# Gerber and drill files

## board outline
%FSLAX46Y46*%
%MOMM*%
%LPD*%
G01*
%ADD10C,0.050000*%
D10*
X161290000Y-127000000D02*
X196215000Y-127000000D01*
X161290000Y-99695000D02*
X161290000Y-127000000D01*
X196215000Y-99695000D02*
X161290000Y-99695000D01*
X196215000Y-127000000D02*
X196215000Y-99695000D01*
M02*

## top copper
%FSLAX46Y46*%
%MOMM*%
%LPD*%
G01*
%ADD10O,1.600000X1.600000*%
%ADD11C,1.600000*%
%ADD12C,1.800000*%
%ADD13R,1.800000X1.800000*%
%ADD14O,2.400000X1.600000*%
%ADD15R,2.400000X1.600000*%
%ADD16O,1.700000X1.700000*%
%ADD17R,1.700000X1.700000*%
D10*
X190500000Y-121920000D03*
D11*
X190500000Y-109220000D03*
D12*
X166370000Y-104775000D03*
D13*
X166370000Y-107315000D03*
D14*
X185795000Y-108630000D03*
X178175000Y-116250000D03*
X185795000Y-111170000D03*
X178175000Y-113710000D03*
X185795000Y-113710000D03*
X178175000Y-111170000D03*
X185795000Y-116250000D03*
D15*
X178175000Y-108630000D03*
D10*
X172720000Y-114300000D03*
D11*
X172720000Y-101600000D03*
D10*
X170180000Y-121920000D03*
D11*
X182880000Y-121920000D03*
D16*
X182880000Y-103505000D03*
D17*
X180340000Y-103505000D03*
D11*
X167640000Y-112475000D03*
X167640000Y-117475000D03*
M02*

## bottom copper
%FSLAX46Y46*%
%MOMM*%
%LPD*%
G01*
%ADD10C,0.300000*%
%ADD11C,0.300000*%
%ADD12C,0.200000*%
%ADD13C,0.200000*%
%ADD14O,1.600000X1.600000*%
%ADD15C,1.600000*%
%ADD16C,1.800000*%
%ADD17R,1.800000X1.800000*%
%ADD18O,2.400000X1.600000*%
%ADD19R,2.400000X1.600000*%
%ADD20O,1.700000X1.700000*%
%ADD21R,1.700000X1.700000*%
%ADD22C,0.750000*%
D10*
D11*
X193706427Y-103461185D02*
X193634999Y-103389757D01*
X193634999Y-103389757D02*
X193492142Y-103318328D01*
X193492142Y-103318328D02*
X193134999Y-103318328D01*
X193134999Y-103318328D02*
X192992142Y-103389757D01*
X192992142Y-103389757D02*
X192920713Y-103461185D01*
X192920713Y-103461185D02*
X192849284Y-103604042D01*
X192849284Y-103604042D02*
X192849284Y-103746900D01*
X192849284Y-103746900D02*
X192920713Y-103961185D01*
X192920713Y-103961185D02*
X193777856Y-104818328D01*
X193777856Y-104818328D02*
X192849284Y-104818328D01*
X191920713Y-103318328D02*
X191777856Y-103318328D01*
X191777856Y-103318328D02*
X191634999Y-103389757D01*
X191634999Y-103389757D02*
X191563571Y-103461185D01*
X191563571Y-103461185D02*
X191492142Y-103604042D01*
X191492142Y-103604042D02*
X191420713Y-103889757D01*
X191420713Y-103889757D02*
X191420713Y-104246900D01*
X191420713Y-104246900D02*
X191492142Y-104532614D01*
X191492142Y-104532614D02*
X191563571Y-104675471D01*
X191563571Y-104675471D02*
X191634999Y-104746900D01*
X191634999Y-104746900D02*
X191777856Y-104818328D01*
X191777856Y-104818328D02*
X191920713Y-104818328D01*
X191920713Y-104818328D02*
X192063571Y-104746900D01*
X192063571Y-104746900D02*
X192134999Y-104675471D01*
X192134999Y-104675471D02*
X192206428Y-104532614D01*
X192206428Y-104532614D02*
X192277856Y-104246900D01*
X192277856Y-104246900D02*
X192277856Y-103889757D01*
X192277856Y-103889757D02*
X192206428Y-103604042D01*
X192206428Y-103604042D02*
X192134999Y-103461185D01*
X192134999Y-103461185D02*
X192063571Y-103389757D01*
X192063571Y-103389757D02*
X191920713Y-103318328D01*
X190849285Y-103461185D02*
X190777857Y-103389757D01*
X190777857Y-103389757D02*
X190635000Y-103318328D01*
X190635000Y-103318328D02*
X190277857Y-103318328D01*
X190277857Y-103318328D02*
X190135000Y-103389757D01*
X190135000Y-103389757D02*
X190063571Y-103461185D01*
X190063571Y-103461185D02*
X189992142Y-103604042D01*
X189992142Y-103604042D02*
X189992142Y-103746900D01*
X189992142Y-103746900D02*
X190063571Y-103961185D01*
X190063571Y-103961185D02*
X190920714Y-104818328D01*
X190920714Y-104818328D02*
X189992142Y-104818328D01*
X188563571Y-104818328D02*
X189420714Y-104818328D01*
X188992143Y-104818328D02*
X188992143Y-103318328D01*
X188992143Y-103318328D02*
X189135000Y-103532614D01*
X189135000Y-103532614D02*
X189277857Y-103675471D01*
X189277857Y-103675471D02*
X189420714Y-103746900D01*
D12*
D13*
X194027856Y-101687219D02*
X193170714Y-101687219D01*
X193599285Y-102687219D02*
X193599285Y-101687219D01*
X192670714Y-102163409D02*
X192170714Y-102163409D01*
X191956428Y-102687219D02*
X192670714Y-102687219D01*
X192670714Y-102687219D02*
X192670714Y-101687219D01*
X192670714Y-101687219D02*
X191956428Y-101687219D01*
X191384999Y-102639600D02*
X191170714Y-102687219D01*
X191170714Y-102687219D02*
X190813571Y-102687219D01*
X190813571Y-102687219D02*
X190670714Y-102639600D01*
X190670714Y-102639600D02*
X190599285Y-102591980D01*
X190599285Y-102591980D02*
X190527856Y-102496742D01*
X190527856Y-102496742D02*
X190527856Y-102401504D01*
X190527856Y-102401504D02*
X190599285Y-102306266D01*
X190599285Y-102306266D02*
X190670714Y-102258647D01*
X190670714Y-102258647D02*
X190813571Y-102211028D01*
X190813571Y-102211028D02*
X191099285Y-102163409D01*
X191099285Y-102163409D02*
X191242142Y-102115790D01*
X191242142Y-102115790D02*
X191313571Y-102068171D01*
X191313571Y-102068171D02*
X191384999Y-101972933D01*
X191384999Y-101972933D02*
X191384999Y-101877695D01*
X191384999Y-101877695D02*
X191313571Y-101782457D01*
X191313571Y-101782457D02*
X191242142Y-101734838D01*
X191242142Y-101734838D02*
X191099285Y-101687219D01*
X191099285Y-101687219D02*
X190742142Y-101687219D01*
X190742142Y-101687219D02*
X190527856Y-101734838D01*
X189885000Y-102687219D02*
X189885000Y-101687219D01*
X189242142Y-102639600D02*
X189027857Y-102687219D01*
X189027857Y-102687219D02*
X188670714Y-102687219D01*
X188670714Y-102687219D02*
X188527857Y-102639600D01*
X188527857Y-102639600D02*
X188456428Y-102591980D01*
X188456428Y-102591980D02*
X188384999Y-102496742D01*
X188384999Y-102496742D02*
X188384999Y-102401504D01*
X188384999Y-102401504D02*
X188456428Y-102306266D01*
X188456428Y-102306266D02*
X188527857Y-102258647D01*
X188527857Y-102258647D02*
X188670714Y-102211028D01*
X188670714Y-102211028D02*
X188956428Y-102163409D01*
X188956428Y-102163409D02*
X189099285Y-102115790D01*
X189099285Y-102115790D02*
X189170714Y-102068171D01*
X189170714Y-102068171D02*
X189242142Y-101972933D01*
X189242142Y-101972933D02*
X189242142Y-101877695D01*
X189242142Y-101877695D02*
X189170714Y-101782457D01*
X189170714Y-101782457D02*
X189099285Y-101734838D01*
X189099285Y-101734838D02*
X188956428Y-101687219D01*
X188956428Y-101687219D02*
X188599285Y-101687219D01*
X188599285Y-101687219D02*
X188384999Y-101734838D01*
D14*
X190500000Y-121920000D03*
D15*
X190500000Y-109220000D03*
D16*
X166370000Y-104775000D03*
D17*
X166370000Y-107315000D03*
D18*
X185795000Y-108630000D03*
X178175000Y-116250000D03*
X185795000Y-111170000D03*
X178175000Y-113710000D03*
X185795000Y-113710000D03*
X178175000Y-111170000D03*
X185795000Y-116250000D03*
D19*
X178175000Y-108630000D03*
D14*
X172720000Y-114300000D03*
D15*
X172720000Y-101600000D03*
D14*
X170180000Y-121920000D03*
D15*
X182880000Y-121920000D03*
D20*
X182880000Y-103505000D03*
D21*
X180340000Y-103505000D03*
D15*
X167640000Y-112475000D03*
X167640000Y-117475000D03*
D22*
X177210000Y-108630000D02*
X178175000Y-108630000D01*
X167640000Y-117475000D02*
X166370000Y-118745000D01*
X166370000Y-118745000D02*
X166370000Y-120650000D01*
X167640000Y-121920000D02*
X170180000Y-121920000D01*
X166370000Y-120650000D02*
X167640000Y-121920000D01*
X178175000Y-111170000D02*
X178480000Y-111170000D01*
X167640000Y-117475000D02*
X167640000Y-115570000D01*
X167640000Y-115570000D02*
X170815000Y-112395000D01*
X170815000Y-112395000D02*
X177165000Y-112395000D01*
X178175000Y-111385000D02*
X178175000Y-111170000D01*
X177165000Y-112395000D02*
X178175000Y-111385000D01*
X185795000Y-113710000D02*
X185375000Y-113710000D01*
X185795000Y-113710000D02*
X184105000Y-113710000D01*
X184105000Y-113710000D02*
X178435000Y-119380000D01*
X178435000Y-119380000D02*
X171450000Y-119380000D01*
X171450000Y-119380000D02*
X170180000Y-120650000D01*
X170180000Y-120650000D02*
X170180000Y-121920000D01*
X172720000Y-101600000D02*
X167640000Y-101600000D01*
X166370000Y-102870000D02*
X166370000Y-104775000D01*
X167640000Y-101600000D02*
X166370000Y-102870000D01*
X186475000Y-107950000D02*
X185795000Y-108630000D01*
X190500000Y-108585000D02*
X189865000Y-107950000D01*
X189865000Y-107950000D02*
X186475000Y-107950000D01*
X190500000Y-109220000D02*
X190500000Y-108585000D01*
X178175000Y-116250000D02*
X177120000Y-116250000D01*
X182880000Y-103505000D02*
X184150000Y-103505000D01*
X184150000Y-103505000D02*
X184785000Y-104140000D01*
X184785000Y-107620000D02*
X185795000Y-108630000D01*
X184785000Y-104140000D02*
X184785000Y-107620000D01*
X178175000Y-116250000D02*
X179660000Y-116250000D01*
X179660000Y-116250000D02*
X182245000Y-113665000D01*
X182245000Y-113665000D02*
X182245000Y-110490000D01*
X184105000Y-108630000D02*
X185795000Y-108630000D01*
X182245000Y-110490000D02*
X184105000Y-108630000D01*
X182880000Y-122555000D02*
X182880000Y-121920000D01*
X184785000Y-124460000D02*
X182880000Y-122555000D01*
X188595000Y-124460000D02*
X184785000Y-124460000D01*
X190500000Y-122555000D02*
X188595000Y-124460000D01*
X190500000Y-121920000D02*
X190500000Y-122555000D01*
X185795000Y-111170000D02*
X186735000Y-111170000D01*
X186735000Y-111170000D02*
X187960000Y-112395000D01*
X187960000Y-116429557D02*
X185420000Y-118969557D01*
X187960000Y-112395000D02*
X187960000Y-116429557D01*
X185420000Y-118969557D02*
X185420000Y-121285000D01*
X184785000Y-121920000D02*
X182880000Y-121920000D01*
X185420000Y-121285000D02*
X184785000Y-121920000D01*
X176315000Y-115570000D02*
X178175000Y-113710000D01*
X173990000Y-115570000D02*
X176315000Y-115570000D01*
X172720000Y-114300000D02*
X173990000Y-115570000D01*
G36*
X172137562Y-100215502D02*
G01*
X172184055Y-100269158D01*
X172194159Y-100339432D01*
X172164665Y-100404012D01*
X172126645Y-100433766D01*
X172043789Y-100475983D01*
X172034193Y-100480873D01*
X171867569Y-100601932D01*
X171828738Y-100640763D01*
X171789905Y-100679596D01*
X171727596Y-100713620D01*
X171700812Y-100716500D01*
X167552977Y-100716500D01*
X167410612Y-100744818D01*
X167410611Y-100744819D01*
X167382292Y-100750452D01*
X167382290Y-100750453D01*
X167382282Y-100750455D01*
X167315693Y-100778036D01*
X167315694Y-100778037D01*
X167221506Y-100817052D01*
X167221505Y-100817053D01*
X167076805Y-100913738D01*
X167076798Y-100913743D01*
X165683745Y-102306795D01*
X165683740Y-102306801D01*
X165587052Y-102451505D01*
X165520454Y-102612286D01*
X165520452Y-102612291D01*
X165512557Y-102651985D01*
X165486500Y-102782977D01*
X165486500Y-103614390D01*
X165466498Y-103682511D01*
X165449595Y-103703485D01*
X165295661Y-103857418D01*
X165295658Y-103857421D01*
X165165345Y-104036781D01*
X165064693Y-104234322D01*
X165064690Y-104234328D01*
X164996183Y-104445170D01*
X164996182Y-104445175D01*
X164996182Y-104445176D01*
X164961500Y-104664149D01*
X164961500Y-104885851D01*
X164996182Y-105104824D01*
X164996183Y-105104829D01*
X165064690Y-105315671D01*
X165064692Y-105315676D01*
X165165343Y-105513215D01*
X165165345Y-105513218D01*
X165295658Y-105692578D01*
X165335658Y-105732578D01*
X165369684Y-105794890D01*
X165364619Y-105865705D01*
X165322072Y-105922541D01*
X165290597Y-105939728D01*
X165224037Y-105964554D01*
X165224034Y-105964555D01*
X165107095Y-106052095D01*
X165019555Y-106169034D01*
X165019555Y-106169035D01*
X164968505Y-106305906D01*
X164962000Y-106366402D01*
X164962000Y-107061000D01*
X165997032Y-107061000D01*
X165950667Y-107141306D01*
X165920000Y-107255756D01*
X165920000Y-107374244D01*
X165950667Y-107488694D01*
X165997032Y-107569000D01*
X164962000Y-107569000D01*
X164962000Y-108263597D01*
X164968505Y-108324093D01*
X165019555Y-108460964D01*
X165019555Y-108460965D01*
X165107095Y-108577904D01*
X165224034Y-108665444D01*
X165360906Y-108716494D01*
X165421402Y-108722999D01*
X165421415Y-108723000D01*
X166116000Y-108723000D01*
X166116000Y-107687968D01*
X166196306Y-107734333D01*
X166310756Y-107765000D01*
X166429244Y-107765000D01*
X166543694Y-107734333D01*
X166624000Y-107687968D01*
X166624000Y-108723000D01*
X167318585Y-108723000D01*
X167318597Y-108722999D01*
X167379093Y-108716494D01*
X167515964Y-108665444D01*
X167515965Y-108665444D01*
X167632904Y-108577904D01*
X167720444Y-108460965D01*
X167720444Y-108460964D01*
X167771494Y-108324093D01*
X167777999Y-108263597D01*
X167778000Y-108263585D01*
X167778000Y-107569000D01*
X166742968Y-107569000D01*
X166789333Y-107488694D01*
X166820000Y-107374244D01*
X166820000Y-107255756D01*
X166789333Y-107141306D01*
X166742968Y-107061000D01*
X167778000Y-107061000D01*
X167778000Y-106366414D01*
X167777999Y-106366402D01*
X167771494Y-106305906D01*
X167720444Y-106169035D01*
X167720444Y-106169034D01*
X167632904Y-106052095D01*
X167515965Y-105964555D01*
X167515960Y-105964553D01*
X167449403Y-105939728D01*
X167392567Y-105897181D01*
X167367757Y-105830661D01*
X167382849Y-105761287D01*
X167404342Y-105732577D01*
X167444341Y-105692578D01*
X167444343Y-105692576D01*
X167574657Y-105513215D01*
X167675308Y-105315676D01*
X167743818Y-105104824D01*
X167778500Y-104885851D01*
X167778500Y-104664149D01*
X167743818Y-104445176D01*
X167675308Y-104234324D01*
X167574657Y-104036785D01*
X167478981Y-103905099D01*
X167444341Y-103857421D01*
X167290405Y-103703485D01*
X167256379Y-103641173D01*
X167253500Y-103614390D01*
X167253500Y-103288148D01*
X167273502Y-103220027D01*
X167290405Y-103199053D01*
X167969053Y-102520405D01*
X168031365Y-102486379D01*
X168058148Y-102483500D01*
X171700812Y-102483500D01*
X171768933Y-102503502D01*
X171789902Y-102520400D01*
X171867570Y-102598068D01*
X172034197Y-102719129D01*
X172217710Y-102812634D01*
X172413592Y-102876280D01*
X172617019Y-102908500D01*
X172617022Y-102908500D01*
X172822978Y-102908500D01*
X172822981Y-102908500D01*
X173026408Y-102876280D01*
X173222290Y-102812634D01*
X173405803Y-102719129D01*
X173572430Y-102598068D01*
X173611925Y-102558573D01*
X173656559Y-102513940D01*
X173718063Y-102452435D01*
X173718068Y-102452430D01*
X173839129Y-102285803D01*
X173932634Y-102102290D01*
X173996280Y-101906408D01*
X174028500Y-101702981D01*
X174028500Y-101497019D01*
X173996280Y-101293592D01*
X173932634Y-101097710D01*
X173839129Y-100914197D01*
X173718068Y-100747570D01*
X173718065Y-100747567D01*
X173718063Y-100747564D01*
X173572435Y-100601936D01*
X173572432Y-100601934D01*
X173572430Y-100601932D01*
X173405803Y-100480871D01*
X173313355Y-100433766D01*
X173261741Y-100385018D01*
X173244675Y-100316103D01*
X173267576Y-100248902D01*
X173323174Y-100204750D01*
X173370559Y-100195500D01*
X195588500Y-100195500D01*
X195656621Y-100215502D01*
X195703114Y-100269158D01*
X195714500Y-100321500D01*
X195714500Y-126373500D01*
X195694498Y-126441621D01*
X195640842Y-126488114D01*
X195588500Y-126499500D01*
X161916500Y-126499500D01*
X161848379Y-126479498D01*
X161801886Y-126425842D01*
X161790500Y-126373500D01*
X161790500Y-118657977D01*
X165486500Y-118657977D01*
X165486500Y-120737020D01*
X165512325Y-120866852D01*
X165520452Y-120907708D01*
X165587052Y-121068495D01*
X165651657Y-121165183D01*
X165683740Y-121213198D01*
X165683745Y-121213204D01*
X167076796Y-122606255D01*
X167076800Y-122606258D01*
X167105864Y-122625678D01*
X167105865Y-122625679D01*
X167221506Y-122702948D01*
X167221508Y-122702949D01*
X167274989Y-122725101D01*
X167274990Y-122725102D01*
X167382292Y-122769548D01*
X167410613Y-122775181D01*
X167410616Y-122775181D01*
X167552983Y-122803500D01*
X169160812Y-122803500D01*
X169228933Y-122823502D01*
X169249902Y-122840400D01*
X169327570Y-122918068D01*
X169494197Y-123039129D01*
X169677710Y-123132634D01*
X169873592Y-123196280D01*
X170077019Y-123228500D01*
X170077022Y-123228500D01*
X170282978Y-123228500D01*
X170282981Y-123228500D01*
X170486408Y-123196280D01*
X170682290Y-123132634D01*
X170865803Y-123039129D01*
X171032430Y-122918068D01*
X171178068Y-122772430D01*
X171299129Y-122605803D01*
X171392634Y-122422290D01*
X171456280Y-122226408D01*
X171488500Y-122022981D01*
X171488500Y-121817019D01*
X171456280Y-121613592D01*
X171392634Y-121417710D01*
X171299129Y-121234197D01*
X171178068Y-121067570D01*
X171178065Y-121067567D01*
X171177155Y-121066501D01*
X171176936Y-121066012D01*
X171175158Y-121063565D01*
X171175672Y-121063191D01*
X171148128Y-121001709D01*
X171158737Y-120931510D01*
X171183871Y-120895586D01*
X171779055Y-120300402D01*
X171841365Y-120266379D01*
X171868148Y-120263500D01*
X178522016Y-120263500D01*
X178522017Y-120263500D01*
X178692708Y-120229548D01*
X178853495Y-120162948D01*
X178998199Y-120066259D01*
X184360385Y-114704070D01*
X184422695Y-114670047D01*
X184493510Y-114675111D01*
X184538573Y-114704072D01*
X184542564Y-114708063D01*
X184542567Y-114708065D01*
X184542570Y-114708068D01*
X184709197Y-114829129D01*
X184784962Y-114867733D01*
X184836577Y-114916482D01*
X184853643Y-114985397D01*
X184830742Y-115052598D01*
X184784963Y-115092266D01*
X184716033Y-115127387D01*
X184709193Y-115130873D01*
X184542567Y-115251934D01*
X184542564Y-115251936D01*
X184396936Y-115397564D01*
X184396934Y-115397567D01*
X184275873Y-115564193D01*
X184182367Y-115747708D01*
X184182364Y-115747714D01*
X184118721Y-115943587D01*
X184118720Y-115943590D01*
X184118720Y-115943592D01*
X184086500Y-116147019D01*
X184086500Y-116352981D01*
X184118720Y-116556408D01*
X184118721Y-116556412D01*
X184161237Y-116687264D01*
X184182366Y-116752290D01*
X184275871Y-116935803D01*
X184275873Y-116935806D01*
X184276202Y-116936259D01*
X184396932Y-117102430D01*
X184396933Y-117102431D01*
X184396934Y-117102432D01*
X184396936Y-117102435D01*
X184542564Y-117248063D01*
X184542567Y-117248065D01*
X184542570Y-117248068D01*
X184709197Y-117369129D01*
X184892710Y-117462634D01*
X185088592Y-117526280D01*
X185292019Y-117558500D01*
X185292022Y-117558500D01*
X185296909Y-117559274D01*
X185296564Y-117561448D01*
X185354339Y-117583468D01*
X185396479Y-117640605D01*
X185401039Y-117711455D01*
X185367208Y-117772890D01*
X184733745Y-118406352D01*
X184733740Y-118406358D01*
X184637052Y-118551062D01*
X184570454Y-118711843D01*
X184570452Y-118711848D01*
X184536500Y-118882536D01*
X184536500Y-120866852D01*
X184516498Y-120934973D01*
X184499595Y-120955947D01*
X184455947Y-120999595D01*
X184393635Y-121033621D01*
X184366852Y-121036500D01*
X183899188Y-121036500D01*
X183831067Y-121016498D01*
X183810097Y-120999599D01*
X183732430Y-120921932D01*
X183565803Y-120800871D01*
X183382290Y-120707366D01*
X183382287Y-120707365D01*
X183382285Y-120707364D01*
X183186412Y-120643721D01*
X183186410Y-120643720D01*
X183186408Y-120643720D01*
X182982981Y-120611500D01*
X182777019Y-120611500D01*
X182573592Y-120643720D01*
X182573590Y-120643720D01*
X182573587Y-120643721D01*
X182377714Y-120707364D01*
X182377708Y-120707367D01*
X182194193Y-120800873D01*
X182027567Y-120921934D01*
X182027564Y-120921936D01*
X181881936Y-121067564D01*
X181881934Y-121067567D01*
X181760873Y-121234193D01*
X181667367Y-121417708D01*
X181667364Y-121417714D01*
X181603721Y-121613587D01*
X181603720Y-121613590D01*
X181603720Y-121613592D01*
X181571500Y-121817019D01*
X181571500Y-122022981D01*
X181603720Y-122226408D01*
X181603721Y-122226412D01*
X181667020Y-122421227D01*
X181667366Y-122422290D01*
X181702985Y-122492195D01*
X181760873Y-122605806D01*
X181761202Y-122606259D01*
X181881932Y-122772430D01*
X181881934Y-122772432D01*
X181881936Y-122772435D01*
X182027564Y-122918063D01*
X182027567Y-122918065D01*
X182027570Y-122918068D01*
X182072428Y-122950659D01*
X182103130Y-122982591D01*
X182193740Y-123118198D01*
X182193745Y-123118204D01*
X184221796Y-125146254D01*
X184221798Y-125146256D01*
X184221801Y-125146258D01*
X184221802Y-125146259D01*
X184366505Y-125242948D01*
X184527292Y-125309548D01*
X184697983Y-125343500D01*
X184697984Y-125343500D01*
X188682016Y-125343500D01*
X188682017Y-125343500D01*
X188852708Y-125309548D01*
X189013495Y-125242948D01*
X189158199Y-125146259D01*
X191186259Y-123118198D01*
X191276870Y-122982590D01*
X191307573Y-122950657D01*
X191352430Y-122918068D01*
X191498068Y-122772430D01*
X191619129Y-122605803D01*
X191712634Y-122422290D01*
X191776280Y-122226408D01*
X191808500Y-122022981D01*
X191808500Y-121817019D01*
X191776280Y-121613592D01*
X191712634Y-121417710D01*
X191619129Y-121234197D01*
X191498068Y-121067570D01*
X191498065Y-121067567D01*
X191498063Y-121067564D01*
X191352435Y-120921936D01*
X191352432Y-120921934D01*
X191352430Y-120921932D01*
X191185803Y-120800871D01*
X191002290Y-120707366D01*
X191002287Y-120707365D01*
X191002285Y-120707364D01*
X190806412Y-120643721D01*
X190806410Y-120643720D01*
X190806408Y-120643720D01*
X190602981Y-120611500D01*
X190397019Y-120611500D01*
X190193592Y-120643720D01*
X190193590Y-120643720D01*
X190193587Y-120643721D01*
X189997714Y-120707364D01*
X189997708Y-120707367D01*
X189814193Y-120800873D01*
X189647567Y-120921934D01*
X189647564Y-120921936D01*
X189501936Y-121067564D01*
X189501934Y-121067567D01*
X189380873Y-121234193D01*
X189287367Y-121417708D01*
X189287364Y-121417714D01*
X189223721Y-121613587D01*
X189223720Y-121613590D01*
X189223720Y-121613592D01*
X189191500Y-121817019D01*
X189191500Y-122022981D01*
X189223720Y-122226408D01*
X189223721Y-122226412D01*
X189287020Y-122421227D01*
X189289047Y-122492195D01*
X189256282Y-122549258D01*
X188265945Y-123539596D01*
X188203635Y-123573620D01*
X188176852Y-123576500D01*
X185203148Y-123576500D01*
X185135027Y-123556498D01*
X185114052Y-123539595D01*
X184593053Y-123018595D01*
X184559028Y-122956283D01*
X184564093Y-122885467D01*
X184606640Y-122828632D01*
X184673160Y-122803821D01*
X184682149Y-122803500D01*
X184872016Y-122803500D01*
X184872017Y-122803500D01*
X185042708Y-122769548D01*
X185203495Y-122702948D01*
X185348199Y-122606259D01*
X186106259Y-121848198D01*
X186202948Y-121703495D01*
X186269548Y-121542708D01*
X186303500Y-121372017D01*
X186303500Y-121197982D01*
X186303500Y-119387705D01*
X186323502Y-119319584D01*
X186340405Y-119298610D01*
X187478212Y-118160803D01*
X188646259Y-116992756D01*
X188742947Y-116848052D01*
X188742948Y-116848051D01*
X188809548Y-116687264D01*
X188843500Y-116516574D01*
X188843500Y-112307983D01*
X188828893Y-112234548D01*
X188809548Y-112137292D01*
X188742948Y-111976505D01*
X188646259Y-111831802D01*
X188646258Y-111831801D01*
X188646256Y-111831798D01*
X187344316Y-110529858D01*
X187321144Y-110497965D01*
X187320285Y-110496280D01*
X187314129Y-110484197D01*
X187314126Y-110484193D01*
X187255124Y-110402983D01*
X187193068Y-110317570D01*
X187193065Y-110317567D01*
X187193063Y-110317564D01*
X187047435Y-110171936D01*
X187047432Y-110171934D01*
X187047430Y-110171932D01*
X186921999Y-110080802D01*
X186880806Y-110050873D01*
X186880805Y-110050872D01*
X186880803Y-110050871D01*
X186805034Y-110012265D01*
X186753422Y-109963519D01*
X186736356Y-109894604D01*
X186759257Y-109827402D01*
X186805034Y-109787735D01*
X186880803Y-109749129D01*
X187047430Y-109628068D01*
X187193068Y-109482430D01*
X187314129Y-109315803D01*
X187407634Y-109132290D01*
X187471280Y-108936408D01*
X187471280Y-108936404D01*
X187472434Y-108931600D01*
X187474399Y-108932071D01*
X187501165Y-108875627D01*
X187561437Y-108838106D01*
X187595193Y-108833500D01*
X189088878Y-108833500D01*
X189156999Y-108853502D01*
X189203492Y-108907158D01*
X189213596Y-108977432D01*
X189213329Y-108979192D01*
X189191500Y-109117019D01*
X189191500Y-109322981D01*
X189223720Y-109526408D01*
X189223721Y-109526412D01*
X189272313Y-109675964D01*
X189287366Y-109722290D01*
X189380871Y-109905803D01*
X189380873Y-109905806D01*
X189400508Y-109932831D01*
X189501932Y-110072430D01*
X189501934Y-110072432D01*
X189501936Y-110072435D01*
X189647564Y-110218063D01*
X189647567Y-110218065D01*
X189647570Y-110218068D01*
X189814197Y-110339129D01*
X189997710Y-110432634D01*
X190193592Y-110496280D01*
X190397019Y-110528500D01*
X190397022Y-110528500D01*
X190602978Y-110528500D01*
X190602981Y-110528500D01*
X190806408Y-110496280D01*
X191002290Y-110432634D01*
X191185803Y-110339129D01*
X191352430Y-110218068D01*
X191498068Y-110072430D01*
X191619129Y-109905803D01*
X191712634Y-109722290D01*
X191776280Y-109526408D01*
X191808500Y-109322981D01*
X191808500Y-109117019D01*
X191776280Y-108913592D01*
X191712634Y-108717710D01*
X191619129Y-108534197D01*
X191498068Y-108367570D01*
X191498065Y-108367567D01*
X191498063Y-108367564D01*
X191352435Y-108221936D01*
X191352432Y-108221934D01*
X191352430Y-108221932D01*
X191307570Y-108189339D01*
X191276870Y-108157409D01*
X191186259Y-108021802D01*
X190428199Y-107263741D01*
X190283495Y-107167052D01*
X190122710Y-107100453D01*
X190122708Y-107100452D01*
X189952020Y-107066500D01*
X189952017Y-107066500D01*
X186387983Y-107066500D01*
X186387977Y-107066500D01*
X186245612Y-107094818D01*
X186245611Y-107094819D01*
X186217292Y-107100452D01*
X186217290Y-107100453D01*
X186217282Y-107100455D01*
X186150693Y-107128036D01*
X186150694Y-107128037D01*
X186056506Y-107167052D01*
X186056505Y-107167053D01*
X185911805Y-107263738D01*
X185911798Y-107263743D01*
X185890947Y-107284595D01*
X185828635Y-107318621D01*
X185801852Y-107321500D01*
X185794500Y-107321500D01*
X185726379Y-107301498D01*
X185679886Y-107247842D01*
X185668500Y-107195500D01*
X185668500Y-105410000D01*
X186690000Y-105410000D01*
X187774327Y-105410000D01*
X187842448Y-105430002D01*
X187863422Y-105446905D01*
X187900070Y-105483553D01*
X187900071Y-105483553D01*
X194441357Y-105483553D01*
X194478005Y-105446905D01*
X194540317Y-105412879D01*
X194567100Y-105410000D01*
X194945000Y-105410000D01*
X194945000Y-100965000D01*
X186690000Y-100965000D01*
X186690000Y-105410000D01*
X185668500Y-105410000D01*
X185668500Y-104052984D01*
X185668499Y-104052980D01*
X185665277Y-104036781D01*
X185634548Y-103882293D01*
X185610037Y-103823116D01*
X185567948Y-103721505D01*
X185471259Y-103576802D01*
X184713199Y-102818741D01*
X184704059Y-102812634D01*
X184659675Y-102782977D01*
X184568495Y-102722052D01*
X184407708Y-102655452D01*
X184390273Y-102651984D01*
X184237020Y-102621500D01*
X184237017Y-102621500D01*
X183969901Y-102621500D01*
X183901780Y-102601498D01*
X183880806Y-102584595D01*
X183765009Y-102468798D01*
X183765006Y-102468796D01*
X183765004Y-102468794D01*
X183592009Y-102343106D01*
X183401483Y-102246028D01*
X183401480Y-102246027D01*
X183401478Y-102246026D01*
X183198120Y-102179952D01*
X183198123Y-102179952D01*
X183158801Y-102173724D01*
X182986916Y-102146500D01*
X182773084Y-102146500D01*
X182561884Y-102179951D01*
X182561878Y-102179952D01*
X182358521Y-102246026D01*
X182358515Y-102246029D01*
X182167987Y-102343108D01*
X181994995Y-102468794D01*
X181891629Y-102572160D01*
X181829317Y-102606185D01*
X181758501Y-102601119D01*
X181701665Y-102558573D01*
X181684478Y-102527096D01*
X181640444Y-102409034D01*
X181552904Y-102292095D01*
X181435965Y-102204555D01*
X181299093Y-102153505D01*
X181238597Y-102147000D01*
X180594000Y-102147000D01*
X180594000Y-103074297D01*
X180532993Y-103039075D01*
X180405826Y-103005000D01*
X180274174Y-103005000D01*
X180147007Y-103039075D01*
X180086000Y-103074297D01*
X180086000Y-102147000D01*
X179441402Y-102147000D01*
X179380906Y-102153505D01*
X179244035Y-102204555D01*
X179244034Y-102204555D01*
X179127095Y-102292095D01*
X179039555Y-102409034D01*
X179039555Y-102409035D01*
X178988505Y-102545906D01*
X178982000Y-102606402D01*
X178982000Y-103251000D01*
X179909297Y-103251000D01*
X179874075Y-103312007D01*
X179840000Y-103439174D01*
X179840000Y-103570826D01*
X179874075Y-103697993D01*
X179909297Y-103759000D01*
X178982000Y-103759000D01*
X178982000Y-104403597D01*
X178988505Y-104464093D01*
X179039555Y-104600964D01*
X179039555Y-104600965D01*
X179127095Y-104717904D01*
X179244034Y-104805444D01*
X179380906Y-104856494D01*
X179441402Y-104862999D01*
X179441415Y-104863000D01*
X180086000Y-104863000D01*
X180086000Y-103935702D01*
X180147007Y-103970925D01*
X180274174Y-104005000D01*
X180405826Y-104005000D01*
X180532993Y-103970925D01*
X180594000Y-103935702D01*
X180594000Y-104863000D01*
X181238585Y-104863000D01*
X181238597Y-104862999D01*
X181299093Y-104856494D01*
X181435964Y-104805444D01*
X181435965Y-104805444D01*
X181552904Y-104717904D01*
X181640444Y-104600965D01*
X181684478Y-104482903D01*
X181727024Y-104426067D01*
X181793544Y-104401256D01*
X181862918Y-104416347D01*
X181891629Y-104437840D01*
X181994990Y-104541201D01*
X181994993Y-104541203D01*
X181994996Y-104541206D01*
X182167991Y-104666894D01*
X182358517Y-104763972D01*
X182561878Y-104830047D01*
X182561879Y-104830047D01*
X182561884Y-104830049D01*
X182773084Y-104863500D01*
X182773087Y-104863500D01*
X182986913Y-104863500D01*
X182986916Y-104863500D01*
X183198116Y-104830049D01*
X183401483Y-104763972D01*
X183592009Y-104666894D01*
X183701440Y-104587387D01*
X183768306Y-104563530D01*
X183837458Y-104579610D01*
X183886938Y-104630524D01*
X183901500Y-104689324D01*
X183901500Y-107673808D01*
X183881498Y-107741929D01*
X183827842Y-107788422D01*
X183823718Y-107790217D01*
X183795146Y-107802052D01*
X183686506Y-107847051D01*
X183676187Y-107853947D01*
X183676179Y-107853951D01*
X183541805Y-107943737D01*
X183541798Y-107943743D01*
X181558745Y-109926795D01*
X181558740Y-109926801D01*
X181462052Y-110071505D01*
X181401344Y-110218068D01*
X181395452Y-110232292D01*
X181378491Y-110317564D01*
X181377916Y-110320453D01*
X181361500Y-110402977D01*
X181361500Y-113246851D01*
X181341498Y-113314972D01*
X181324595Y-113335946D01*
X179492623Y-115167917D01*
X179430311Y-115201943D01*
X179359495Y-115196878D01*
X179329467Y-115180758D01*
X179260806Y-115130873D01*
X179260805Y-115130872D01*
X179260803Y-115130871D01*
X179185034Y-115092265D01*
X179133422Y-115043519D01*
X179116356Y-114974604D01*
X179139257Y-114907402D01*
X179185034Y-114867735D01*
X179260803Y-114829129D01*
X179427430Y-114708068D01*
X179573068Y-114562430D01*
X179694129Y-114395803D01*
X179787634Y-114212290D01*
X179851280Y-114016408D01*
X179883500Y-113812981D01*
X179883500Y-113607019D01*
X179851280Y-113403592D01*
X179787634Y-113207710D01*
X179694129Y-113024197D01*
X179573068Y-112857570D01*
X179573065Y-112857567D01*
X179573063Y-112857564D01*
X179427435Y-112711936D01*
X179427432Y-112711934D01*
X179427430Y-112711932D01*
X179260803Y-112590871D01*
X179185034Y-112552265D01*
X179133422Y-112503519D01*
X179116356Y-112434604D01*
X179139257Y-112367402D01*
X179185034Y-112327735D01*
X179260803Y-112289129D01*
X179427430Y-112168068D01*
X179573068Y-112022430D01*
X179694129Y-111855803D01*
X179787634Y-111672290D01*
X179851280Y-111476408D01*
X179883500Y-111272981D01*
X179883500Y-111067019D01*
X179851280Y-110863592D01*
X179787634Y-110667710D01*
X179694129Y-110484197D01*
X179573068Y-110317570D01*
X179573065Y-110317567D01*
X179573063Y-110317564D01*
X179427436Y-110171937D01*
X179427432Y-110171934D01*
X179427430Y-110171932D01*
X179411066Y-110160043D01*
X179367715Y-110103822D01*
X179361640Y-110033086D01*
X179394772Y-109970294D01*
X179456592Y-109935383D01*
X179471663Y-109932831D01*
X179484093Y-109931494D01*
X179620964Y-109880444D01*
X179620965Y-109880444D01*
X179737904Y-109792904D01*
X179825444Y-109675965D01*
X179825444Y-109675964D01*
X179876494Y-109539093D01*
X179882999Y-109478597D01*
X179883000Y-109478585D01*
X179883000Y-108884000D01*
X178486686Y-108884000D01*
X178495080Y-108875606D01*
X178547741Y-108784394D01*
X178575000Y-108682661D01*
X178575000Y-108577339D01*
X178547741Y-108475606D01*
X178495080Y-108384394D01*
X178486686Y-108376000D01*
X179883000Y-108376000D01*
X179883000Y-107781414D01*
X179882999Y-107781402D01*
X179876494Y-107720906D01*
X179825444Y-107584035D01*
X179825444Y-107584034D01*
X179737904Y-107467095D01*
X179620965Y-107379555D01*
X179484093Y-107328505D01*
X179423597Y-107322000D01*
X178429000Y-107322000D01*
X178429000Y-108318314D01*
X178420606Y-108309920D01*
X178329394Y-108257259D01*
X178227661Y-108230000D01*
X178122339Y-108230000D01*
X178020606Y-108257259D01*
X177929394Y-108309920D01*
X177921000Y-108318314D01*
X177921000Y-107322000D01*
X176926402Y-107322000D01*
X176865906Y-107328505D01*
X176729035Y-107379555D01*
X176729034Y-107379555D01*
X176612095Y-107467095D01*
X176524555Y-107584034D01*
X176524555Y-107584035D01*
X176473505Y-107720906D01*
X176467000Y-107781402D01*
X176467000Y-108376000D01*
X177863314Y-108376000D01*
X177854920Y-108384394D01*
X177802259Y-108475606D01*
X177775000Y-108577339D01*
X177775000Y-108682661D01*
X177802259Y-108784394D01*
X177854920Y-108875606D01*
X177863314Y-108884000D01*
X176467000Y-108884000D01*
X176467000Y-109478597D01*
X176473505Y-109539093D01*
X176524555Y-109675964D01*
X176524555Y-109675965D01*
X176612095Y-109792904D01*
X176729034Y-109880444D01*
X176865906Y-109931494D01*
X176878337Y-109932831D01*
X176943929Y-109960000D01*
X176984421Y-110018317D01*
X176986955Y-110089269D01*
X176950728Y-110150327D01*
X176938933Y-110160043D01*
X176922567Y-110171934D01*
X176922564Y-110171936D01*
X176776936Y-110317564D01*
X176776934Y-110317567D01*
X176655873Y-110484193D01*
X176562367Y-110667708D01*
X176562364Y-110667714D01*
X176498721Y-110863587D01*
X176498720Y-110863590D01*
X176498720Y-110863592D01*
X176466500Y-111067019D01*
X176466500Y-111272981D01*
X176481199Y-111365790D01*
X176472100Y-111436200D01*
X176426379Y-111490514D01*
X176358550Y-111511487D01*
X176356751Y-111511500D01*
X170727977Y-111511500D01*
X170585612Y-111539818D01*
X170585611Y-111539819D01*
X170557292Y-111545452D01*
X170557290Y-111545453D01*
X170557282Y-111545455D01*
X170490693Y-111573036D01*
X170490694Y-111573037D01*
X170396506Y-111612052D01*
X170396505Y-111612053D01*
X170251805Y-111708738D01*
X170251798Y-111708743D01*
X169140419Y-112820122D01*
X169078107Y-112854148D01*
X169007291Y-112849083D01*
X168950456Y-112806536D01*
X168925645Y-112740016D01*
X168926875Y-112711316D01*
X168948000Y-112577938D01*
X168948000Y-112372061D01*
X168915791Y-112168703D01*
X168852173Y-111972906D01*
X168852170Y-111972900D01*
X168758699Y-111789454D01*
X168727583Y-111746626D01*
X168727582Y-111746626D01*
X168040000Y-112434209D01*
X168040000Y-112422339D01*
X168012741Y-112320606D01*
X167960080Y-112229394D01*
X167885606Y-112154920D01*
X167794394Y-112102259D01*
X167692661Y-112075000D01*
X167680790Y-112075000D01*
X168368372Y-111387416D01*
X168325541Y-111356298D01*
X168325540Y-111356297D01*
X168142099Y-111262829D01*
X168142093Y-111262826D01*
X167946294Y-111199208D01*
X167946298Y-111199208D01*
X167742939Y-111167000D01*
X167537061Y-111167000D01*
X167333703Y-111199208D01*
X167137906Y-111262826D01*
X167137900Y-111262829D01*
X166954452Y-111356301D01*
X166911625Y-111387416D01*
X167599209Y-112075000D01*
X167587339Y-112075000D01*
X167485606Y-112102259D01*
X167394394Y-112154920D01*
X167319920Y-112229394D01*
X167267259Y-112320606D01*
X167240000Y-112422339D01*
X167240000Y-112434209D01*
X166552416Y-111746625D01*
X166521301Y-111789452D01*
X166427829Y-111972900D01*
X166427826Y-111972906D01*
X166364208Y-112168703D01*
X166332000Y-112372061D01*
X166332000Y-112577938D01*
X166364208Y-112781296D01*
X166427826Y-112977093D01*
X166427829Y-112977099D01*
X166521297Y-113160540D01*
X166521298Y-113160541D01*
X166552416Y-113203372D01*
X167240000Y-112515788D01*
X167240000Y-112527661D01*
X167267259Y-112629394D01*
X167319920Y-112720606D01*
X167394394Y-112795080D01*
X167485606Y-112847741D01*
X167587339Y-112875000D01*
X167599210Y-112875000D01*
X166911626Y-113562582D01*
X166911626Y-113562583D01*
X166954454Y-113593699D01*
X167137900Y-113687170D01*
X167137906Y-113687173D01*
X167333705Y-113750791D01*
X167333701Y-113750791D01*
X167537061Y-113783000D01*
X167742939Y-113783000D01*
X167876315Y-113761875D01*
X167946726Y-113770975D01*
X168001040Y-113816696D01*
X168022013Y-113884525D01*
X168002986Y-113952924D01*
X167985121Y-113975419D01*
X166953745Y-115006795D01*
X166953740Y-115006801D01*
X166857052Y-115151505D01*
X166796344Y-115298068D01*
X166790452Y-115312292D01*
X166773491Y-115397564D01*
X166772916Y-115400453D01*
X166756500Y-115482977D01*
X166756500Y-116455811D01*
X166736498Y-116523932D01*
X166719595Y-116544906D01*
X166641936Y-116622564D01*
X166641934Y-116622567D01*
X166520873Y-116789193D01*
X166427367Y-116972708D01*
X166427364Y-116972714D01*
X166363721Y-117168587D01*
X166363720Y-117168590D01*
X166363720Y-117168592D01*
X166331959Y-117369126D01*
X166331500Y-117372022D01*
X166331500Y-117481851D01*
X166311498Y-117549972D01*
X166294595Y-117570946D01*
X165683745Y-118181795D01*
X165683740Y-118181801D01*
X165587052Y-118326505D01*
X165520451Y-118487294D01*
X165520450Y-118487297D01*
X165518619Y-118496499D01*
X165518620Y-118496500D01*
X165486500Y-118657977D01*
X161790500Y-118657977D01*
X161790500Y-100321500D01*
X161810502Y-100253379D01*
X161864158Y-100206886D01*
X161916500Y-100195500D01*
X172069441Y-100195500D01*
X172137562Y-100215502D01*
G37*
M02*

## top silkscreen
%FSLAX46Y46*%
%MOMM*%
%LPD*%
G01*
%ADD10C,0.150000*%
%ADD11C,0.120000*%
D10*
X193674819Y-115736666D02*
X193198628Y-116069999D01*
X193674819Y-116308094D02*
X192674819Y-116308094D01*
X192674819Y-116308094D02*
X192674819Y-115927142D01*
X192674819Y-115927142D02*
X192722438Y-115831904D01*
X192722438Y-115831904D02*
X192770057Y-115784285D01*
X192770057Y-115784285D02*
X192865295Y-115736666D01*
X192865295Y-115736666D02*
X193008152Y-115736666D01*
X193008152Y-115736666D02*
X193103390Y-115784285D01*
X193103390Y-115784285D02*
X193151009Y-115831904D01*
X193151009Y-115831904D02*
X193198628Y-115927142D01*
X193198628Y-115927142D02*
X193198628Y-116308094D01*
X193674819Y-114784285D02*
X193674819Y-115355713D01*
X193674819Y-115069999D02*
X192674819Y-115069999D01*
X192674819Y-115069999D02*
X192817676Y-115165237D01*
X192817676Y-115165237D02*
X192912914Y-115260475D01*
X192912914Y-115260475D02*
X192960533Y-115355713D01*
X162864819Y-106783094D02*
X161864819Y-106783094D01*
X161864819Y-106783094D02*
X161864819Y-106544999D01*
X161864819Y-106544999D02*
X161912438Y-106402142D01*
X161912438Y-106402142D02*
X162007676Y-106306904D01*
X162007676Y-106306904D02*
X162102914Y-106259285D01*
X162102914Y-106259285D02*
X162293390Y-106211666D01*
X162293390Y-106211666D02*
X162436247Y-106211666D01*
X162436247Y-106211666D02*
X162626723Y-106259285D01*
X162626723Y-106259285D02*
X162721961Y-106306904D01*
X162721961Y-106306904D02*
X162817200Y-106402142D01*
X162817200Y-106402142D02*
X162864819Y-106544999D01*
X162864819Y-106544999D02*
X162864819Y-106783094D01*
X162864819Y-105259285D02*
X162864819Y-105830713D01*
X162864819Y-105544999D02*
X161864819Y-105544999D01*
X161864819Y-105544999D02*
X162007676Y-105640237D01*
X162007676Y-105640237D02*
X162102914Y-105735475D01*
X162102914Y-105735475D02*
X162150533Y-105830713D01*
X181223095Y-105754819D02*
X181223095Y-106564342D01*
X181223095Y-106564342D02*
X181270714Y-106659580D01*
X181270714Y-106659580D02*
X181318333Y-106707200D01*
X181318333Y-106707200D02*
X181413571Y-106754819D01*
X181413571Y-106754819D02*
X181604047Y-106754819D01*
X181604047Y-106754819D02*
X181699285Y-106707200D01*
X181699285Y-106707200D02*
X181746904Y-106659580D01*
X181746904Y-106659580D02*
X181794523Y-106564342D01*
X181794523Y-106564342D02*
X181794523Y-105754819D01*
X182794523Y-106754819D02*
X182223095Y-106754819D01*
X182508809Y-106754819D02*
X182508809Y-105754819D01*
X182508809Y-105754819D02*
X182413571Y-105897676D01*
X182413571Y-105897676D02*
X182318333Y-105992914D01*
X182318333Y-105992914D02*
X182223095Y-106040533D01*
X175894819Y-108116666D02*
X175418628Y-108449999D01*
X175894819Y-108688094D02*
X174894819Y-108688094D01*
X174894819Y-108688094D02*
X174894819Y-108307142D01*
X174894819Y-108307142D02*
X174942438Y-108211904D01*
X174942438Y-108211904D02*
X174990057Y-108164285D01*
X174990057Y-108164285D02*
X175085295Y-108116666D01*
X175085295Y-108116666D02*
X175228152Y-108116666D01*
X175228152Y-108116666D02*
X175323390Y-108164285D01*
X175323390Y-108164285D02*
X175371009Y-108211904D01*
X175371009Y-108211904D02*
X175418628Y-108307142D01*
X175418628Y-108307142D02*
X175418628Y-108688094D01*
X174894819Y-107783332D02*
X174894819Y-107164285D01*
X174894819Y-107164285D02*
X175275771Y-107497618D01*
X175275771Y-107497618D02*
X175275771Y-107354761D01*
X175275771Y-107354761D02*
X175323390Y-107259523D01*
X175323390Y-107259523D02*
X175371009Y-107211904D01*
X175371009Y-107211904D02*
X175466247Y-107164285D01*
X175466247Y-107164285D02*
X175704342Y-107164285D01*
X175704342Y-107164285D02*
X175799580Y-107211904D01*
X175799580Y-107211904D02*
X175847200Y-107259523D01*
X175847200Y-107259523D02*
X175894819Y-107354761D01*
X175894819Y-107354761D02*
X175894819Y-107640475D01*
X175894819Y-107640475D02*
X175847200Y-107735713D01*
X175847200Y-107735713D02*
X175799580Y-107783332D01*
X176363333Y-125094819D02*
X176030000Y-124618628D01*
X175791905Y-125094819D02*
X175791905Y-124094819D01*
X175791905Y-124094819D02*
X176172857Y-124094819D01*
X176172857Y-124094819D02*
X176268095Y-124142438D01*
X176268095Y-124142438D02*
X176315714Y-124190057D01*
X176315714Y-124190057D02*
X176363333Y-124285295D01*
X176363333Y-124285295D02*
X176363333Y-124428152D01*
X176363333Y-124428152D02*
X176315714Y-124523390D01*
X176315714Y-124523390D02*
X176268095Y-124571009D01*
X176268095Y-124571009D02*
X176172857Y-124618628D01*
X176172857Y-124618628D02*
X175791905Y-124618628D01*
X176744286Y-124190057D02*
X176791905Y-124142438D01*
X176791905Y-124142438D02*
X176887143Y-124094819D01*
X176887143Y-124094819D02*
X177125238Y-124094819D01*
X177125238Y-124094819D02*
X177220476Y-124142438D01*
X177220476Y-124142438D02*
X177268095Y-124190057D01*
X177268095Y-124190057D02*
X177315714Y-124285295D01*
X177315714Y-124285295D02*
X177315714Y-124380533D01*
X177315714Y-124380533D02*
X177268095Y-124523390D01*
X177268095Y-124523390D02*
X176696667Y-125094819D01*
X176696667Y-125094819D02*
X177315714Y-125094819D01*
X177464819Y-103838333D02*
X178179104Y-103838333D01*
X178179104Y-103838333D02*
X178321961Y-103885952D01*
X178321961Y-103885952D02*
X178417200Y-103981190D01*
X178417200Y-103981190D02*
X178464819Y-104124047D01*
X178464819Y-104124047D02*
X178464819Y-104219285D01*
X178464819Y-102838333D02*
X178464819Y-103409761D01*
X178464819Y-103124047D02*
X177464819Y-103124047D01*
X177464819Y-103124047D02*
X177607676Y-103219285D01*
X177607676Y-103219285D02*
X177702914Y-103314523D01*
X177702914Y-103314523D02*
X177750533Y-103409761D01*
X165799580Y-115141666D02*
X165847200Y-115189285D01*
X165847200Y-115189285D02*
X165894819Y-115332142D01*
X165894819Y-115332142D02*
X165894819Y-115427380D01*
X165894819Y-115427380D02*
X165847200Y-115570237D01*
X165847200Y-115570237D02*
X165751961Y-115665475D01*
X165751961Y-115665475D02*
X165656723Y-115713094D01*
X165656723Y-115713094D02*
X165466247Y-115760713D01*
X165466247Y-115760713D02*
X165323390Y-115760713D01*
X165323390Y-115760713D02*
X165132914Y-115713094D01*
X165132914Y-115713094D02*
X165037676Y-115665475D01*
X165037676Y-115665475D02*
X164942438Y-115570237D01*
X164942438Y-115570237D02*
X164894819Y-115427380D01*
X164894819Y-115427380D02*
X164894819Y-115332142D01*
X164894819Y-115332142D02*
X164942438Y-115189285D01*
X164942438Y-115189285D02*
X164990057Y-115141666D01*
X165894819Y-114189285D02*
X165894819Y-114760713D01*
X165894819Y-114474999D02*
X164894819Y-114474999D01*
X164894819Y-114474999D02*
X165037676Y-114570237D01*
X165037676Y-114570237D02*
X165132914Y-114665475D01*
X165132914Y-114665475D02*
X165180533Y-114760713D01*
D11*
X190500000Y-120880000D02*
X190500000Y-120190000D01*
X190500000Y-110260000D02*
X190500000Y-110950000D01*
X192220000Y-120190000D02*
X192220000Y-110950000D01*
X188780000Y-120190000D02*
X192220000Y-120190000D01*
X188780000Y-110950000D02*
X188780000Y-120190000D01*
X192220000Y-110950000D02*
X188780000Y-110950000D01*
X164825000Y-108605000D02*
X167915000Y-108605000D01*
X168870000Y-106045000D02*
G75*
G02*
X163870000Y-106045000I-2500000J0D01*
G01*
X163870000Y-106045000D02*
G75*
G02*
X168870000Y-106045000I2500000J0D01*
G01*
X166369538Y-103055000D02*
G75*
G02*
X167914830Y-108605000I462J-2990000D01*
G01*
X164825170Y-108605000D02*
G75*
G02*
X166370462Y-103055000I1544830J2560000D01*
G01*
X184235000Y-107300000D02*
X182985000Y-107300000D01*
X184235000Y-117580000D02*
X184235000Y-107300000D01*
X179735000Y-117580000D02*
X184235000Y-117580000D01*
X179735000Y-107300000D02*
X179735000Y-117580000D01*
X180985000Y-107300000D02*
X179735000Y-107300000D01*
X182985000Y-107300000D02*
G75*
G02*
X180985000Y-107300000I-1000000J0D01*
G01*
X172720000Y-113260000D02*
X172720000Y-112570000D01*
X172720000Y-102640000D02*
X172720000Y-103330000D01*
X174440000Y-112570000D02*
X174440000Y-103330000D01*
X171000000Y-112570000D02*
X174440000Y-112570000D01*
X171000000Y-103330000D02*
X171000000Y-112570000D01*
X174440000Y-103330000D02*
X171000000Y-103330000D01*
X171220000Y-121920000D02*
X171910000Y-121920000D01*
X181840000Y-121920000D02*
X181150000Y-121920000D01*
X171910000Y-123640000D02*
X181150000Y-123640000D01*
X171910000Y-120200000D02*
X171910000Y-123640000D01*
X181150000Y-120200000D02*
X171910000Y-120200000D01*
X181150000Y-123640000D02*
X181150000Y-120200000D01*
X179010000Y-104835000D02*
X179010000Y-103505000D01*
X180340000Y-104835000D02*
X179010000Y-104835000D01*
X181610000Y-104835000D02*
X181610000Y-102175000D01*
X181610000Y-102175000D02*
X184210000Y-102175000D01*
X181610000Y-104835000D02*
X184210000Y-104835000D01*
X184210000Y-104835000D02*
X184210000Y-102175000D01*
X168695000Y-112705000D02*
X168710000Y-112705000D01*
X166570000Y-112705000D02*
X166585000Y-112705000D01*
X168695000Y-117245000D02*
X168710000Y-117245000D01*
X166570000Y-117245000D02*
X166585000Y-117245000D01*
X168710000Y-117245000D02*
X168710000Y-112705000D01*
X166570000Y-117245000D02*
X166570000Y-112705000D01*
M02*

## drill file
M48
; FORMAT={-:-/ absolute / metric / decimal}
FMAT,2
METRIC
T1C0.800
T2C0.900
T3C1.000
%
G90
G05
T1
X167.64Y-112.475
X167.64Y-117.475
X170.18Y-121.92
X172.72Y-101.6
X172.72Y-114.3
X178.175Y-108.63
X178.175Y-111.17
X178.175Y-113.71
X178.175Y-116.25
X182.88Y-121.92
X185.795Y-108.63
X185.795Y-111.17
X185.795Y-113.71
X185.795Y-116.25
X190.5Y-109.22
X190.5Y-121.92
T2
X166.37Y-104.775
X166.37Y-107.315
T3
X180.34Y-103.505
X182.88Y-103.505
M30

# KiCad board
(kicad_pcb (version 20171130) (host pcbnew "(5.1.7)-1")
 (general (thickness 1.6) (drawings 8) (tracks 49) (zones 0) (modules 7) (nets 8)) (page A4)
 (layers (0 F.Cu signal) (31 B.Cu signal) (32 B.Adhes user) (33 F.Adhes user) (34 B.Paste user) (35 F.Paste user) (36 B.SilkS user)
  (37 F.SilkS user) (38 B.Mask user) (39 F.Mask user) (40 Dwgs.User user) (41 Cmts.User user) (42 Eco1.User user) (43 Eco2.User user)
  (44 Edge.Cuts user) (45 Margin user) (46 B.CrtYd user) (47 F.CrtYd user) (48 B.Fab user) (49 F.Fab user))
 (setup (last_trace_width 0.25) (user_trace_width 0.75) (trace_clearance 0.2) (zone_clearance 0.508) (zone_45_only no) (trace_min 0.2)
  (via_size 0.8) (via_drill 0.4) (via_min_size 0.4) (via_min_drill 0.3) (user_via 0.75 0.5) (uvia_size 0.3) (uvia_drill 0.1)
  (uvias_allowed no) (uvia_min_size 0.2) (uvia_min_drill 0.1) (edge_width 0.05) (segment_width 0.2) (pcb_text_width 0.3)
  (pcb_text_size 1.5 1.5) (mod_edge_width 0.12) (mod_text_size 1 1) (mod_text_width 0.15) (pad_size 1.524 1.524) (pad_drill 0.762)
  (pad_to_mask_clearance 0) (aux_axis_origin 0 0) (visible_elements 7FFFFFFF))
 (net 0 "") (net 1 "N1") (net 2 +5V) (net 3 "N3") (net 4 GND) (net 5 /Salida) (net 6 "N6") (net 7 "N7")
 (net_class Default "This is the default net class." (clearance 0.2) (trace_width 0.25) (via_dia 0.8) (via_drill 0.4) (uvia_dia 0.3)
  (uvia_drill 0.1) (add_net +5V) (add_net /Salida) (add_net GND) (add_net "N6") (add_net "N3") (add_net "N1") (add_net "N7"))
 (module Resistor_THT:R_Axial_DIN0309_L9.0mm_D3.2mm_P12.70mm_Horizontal (layer F.Cu) (at 190.5 109.22 270)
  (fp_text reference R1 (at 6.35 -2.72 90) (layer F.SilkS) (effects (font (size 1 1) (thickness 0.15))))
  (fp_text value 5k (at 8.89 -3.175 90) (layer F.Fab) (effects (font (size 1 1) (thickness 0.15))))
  (fp_line (start 11.66 0) (end 10.97 0) (layer F.SilkS) (width 0.12))
  (fp_line (start 1.04 0) (end 1.73 0) (layer F.SilkS) (width 0.12))
  (fp_line (start 10.97 -1.72) (end 1.73 -1.72) (layer F.SilkS) (width 0.12))
  (fp_line (start 10.97 1.72) (end 10.97 -1.72) (layer F.SilkS) (width 0.12))
  (fp_line (start 1.73 1.72) (end 10.97 1.72) (layer F.SilkS) (width 0.12))
  (fp_line (start 1.73 -1.72) (end 1.73 1.72) (layer F.SilkS) (width 0.12))
  (pad 2 thru_hole oval (at 12.7 0 270) (size 1.6 1.6) (drill 0.8) (layers *.Cu *.Mask) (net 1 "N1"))
  (pad 1 thru_hole circle (at 0 0 270) (size 1.6 1.6) (drill 0.8) (layers *.Cu *.Mask) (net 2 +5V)))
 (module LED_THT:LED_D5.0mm (layer F.Cu) (at 166.37 107.315 90)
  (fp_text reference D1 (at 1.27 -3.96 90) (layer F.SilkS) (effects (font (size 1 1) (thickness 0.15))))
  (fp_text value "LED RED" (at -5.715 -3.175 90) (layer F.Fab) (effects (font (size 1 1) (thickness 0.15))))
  (fp_line (start -1.29 -1.545) (end -1.29 1.545) (layer F.SilkS) (width 0.12))
  (fp_circle (center 1.27 0) (end 3.77 0) (layer F.SilkS) (width 0.12))
  (fp_arc (start 1.27 0) (end -1.29 1.54483) (angle -148.9) (layer F.SilkS) (width 0.12))
  (fp_arc (start 1.27 0) (end -1.29 -1.54483) (angle 148.9) (layer F.SilkS) (width 0.12))
  (pad 2 thru_hole circle (at 2.54 0 90) (size 1.8 1.8) (drill 0.9) (layers *.Cu *.Mask) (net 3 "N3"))
  (pad 1 thru_hole rect (at 0 0 90) (size 1.8 1.8) (drill 0.9) (layers *.Cu *.Mask) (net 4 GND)))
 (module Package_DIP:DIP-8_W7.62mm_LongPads (layer F.Cu) (at 178.175 108.63)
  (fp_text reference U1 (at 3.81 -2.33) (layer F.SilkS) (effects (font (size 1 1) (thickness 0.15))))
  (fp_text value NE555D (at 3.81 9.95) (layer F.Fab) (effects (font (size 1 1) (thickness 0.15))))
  (fp_line (start 6.06 -1.33) (end 4.81 -1.33) (layer F.SilkS) (width 0.12))
  (fp_line (start 6.06 8.95) (end 6.06 -1.33) (layer F.SilkS) (width 0.12))
  (fp_line (start 1.56 8.95) (end 6.06 8.95) (layer F.SilkS) (width 0.12))
  (fp_line (start 1.56 -1.33) (end 1.56 8.95) (layer F.SilkS) (width 0.12))
  (fp_line (start 2.81 -1.33) (end 1.56 -1.33) (layer F.SilkS) (width 0.12))
  (fp_arc (start 3.81 -1.33) (end 2.81 -1.33) (angle -180) (layer F.SilkS) (width 0.12))
  (pad 8 thru_hole oval (at 7.62 0) (size 2.4 1.6) (drill 0.8) (layers *.Cu *.Mask) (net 2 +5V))
  (pad 4 thru_hole oval (at 0 7.62) (size 2.4 1.6) (drill 0.8) (layers *.Cu *.Mask) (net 2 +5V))
  (pad 7 thru_hole oval (at 7.62 2.54) (size 2.4 1.6) (drill 0.8) (layers *.Cu *.Mask) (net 1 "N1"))
  (pad 3 thru_hole oval (at 0 5.08) (size 2.4 1.6) (drill 0.8) (layers *.Cu *.Mask) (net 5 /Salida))
  (pad 6 thru_hole oval (at 7.62 5.08) (size 2.4 1.6) (drill 0.8) (layers *.Cu *.Mask) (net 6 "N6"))
  (pad 2 thru_hole oval (at 0 2.54) (size 2.4 1.6) (drill 0.8) (layers *.Cu *.Mask) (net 6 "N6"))
  (pad 5 thru_hole oval (at 7.62 7.62) (size 2.4 1.6) (drill 0.8) (layers *.Cu *.Mask) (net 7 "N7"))
  (pad 1 thru_hole rect (at 0 0) (size 2.4 1.6) (drill 0.8) (layers *.Cu *.Mask) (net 4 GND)))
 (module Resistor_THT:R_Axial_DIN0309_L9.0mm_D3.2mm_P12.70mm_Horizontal (layer F.Cu) (at 172.72 101.6 270)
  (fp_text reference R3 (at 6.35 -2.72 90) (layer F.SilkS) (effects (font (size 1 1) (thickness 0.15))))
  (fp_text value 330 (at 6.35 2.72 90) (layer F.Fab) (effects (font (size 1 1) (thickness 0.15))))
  (fp_line (start 11.66 0) (end 10.97 0) (layer F.SilkS) (width 0.12))
  (fp_line (start 1.04 0) (end 1.73 0) (layer F.SilkS) (width 0.12))
  (fp_line (start 10.97 -1.72) (end 1.73 -1.72) (layer F.SilkS) (width 0.12))
  (fp_line (start 10.97 1.72) (end 10.97 -1.72) (layer F.SilkS) (width 0.12))
  (fp_line (start 1.73 1.72) (end 10.97 1.72) (layer F.SilkS) (width 0.12))
  (fp_line (start 1.73 -1.72) (end 1.73 1.72) (layer F.SilkS) (width 0.12))
  (pad 2 thru_hole oval (at 12.7 0 270) (size 1.6 1.6) (drill 0.8) (layers *.Cu *.Mask) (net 5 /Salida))
  (pad 1 thru_hole circle (at 0 0 270) (size 1.6 1.6) (drill 0.8) (layers *.Cu *.Mask) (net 3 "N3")))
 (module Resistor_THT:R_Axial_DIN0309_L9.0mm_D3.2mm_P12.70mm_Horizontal (layer F.Cu) (at 182.88 121.92 180)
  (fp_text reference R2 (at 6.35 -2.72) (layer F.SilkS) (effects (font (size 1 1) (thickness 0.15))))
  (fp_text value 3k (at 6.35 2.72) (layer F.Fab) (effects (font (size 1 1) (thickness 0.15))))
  (fp_line (start 11.66 0) (end 10.97 0) (layer F.SilkS) (width 0.12))
  (fp_line (start 1.04 0) (end 1.73 0) (layer F.SilkS) (width 0.12))
  (fp_line (start 10.97 -1.72) (end 1.73 -1.72) (layer F.SilkS) (width 0.12))
  (fp_line (start 10.97 1.72) (end 10.97 -1.72) (layer F.SilkS) (width 0.12))
  (fp_line (start 1.73 1.72) (end 10.97 1.72) (layer F.SilkS) (width 0.12))
  (fp_line (start 1.73 -1.72) (end 1.73 1.72) (layer F.SilkS) (width 0.12))
  (pad 2 thru_hole oval (at 12.7 0 180) (size 1.6 1.6) (drill 0.8) (layers *.Cu *.Mask) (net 6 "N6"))
  (pad 1 thru_hole circle (at 0 0 180) (size 1.6 1.6) (drill 0.8) (layers *.Cu *.Mask) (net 1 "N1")))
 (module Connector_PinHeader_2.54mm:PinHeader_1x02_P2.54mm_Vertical (layer F.Cu) (at 180.34 103.505 90)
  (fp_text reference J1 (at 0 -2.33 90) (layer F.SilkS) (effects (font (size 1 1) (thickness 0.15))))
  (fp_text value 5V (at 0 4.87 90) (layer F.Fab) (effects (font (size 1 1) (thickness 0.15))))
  (fp_line (start -1.33 -1.33) (end 0 -1.33) (layer F.SilkS) (width 0.12))
  (fp_line (start -1.33 0) (end -1.33 -1.33) (layer F.SilkS) (width 0.12))
  (fp_line (start -1.33 1.27) (end 1.33 1.27) (layer F.SilkS) (width 0.12))
  (fp_line (start 1.33 1.27) (end 1.33 3.87) (layer F.SilkS) (width 0.12))
  (fp_line (start -1.33 1.27) (end -1.33 3.87) (layer F.SilkS) (width 0.12))
  (fp_line (start -1.33 3.87) (end 1.33 3.87) (layer F.SilkS) (width 0.12))
  (pad 2 thru_hole oval (at 0 2.54 90) (size 1.7 1.7) (drill 1) (layers *.Cu *.Mask) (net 2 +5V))
  (pad 1 thru_hole rect (at 0 0 90) (size 1.7 1.7) (drill 1) (layers *.Cu *.Mask) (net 4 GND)))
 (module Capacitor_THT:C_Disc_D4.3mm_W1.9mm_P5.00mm (layer F.Cu) (at 167.64 117.475 90)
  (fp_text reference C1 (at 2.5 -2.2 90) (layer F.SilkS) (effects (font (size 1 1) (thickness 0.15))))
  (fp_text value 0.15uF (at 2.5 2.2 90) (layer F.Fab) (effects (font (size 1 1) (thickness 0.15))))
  (fp_line (start 4.77 1.055) (end 4.77 1.07) (layer F.SilkS) (width 0.12))
  (fp_line (start 4.77 -1.07) (end 4.77 -1.055) (layer F.SilkS) (width 0.12))
  (fp_line (start 0.23 1.055) (end 0.23 1.07) (layer F.SilkS) (width 0.12))
  (fp_line (start 0.23 -1.07) (end 0.23 -1.055) (layer F.SilkS) (width 0.12))
  (fp_line (start 0.23 1.07) (end 4.77 1.07) (layer F.SilkS) (width 0.12))
  (fp_line (start 0.23 -1.07) (end 4.77 -1.07) (layer F.SilkS) (width 0.12))
  (pad 2 thru_hole circle (at 5 0 90) (size 1.6 1.6) (drill 0.8) (layers *.Cu *.Mask) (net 4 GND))
  (pad 1 thru_hole circle (at 0 0 90) (size 1.6 1.6) (drill 0.8) (layers *.Cu *.Mask) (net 6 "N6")))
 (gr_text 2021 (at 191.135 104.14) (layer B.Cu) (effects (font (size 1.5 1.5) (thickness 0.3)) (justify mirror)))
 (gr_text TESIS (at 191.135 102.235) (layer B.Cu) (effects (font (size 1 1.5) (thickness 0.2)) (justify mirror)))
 (gr_line (start 161.29 127) (end 196.215 127) (layer Edge.Cuts) (width 0.05))
 (gr_line (start 161.29 99.695) (end 161.29 127) (layer Edge.Cuts) (width 0.05))
 (gr_line (start 196.215 99.695) (end 161.29 99.695) (layer Edge.Cuts) (width 0.05))
 (gr_line (start 196.215 127) (end 196.215 99.695) (layer Edge.Cuts) (width 0.05))
 (segment (start 177.21 108.63) (end 178.175 108.63) (width 0.75) (layer B.Cu) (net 4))
 (segment (start 167.64 117.475) (end 166.37 118.745) (width 0.75) (layer B.Cu) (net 6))
 (segment (start 166.37 118.745) (end 166.37 120.65) (width 0.75) (layer B.Cu) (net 6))
 (segment (start 167.64 121.92) (end 170.18 121.92) (width 0.75) (layer B.Cu) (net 6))
 (segment (start 166.37 120.65) (end 167.64 121.92) (width 0.75) (layer B.Cu) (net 6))
 (segment (start 178.175 111.17) (end 178.48 111.17) (width 0.75) (layer B.Cu) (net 6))
 (segment (start 167.64 117.475) (end 167.64 115.57) (width 0.75) (layer B.Cu) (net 6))
 (segment (start 167.64 115.57) (end 170.815 112.395) (width 0.75) (layer B.Cu) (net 6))
 (segment (start 170.815 112.395) (end 177.165 112.395) (width 0.75) (layer B.Cu) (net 6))
 (segment (start 178.175 111.385) (end 178.175 111.17) (width 0.75) (layer B.Cu) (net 6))
 (segment (start 177.165 112.395) (end 178.175 111.385) (width 0.75) (layer B.Cu) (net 6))
 (segment (start 185.795 113.71) (end 185.375 113.71) (width 0.75) (layer B.Cu) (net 6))
 (segment (start 185.795 113.71) (end 184.105 113.71) (width 0.75) (layer B.Cu) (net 6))
 (segment (start 184.105 113.71) (end 178.435 119.38) (width 0.75) (layer B.Cu) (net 6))
 (segment (start 178.435 119.38) (end 171.45 119.38) (width 0.75) (layer B.Cu) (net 6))
 (segment (start 171.45 119.38) (end 170.18 120.65) (width 0.75) (layer B.Cu) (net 6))
 (segment (start 170.18 120.65) (end 170.18 121.92) (width 0.75) (layer B.Cu) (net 6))
 (segment (start 172.72 101.6) (end 167.64 101.6) (width 0.75) (layer B.Cu) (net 3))
 (segment (start 166.37 102.87) (end 166.37 104.775) (width 0.75) (layer B.Cu) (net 3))
 (segment (start 167.64 101.6) (end 166.37 102.87) (width 0.75) (layer B.Cu) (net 3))
 (segment (start 186.475 107.95) (end 185.795 108.63) (width 0.75) (layer B.Cu) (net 2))
 (segment (start 190.5 108.585) (end 189.865 107.95) (width 0.75) (layer B.Cu) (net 2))
 (segment (start 189.865 107.95) (end 186.475 107.95) (width 0.75) (layer B.Cu) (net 2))
 (segment (start 190.5 109.22) (end 190.5 108.585) (width 0.75) (layer B.Cu) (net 2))
 (segment (start 178.175 116.25) (end 177.12 116.25) (width 0.75) (layer B.Cu) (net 2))
 (segment (start 182.88 103.505) (end 184.15 103.505) (width 0.75) (layer B.Cu) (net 2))
 (segment (start 184.15 103.505) (end 184.785 104.14) (width 0.75) (layer B.Cu) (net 2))
 (segment (start 184.785 107.62) (end 185.795 108.63) (width 0.75) (layer B.Cu) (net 2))
 (segment (start 184.785 104.14) (end 184.785 107.62) (width 0.75) (layer B.Cu) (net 2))
 (segment (start 178.175 116.25) (end 179.66 116.25) (width 0.75) (layer B.Cu) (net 2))
 (segment (start 179.66 116.25) (end 182.245 113.665) (width 0.75) (layer B.Cu) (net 2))
 (segment (start 182.245 113.665) (end 182.245 110.49) (width 0.75) (layer B.Cu) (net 2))
 (segment (start 184.105 108.63) (end 185.795 108.63) (width 0.75) (layer B.Cu) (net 2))
 (segment (start 182.245 110.49) (end 184.105 108.63) (width 0.75) (layer B.Cu) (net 2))
 (segment (start 182.88 122.555) (end 182.88 121.92) (width 0.75) (layer B.Cu) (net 1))
 (segment (start 184.785 124.46) (end 182.88 122.555) (width 0.75) (layer B.Cu) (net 1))
 (segment (start 188.595 124.46) (end 184.785 124.46) (width 0.75) (layer B.Cu) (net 1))
 (segment (start 190.5 122.555) (end 188.595 124.46) (width 0.75) (layer B.Cu) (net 1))
 (segment (start 190.5 121.92) (end 190.5 122.555) (width 0.75) (layer B.Cu) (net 1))
 (segment (start 185.795 111.17) (end 186.735 111.17) (width 0.75) (layer B.Cu) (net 1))
 (segment (start 186.735 111.17) (end 187.96 112.395) (width 0.75) (layer B.Cu) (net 1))
 (segment (start 187.96 116.429557) (end 185.42 118.969557) (width 0.75) (layer B.Cu) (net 1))
 (segment (start 187.96 112.395) (end 187.96 116.429557) (width 0.75) (layer B.Cu) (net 1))
 (segment (start 185.42 118.969557) (end 185.42 121.285) (width 0.75) (layer B.Cu) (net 1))
 (segment (start 184.785 121.92) (end 182.88 121.92) (width 0.75) (layer B.Cu) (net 1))
 (segment (start 185.42 121.285) (end 184.785 121.92) (width 0.75) (layer B.Cu) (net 1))
 (segment (start 176.315 115.57) (end 178.175 113.71) (width 0.75) (layer B.Cu) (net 5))
 (segment (start 173.99 115.57) (end 176.315 115.57) (width 0.75) (layer B.Cu) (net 5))
 (segment (start 172.72 114.3) (end 173.99 115.57) (width 0.75) (layer B.Cu) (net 5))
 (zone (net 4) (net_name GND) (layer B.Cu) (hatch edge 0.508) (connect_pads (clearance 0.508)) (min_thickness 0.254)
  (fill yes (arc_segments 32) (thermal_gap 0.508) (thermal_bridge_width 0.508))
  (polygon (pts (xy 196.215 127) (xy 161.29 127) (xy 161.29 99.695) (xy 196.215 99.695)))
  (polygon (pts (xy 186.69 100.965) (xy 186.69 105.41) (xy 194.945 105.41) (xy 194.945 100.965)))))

